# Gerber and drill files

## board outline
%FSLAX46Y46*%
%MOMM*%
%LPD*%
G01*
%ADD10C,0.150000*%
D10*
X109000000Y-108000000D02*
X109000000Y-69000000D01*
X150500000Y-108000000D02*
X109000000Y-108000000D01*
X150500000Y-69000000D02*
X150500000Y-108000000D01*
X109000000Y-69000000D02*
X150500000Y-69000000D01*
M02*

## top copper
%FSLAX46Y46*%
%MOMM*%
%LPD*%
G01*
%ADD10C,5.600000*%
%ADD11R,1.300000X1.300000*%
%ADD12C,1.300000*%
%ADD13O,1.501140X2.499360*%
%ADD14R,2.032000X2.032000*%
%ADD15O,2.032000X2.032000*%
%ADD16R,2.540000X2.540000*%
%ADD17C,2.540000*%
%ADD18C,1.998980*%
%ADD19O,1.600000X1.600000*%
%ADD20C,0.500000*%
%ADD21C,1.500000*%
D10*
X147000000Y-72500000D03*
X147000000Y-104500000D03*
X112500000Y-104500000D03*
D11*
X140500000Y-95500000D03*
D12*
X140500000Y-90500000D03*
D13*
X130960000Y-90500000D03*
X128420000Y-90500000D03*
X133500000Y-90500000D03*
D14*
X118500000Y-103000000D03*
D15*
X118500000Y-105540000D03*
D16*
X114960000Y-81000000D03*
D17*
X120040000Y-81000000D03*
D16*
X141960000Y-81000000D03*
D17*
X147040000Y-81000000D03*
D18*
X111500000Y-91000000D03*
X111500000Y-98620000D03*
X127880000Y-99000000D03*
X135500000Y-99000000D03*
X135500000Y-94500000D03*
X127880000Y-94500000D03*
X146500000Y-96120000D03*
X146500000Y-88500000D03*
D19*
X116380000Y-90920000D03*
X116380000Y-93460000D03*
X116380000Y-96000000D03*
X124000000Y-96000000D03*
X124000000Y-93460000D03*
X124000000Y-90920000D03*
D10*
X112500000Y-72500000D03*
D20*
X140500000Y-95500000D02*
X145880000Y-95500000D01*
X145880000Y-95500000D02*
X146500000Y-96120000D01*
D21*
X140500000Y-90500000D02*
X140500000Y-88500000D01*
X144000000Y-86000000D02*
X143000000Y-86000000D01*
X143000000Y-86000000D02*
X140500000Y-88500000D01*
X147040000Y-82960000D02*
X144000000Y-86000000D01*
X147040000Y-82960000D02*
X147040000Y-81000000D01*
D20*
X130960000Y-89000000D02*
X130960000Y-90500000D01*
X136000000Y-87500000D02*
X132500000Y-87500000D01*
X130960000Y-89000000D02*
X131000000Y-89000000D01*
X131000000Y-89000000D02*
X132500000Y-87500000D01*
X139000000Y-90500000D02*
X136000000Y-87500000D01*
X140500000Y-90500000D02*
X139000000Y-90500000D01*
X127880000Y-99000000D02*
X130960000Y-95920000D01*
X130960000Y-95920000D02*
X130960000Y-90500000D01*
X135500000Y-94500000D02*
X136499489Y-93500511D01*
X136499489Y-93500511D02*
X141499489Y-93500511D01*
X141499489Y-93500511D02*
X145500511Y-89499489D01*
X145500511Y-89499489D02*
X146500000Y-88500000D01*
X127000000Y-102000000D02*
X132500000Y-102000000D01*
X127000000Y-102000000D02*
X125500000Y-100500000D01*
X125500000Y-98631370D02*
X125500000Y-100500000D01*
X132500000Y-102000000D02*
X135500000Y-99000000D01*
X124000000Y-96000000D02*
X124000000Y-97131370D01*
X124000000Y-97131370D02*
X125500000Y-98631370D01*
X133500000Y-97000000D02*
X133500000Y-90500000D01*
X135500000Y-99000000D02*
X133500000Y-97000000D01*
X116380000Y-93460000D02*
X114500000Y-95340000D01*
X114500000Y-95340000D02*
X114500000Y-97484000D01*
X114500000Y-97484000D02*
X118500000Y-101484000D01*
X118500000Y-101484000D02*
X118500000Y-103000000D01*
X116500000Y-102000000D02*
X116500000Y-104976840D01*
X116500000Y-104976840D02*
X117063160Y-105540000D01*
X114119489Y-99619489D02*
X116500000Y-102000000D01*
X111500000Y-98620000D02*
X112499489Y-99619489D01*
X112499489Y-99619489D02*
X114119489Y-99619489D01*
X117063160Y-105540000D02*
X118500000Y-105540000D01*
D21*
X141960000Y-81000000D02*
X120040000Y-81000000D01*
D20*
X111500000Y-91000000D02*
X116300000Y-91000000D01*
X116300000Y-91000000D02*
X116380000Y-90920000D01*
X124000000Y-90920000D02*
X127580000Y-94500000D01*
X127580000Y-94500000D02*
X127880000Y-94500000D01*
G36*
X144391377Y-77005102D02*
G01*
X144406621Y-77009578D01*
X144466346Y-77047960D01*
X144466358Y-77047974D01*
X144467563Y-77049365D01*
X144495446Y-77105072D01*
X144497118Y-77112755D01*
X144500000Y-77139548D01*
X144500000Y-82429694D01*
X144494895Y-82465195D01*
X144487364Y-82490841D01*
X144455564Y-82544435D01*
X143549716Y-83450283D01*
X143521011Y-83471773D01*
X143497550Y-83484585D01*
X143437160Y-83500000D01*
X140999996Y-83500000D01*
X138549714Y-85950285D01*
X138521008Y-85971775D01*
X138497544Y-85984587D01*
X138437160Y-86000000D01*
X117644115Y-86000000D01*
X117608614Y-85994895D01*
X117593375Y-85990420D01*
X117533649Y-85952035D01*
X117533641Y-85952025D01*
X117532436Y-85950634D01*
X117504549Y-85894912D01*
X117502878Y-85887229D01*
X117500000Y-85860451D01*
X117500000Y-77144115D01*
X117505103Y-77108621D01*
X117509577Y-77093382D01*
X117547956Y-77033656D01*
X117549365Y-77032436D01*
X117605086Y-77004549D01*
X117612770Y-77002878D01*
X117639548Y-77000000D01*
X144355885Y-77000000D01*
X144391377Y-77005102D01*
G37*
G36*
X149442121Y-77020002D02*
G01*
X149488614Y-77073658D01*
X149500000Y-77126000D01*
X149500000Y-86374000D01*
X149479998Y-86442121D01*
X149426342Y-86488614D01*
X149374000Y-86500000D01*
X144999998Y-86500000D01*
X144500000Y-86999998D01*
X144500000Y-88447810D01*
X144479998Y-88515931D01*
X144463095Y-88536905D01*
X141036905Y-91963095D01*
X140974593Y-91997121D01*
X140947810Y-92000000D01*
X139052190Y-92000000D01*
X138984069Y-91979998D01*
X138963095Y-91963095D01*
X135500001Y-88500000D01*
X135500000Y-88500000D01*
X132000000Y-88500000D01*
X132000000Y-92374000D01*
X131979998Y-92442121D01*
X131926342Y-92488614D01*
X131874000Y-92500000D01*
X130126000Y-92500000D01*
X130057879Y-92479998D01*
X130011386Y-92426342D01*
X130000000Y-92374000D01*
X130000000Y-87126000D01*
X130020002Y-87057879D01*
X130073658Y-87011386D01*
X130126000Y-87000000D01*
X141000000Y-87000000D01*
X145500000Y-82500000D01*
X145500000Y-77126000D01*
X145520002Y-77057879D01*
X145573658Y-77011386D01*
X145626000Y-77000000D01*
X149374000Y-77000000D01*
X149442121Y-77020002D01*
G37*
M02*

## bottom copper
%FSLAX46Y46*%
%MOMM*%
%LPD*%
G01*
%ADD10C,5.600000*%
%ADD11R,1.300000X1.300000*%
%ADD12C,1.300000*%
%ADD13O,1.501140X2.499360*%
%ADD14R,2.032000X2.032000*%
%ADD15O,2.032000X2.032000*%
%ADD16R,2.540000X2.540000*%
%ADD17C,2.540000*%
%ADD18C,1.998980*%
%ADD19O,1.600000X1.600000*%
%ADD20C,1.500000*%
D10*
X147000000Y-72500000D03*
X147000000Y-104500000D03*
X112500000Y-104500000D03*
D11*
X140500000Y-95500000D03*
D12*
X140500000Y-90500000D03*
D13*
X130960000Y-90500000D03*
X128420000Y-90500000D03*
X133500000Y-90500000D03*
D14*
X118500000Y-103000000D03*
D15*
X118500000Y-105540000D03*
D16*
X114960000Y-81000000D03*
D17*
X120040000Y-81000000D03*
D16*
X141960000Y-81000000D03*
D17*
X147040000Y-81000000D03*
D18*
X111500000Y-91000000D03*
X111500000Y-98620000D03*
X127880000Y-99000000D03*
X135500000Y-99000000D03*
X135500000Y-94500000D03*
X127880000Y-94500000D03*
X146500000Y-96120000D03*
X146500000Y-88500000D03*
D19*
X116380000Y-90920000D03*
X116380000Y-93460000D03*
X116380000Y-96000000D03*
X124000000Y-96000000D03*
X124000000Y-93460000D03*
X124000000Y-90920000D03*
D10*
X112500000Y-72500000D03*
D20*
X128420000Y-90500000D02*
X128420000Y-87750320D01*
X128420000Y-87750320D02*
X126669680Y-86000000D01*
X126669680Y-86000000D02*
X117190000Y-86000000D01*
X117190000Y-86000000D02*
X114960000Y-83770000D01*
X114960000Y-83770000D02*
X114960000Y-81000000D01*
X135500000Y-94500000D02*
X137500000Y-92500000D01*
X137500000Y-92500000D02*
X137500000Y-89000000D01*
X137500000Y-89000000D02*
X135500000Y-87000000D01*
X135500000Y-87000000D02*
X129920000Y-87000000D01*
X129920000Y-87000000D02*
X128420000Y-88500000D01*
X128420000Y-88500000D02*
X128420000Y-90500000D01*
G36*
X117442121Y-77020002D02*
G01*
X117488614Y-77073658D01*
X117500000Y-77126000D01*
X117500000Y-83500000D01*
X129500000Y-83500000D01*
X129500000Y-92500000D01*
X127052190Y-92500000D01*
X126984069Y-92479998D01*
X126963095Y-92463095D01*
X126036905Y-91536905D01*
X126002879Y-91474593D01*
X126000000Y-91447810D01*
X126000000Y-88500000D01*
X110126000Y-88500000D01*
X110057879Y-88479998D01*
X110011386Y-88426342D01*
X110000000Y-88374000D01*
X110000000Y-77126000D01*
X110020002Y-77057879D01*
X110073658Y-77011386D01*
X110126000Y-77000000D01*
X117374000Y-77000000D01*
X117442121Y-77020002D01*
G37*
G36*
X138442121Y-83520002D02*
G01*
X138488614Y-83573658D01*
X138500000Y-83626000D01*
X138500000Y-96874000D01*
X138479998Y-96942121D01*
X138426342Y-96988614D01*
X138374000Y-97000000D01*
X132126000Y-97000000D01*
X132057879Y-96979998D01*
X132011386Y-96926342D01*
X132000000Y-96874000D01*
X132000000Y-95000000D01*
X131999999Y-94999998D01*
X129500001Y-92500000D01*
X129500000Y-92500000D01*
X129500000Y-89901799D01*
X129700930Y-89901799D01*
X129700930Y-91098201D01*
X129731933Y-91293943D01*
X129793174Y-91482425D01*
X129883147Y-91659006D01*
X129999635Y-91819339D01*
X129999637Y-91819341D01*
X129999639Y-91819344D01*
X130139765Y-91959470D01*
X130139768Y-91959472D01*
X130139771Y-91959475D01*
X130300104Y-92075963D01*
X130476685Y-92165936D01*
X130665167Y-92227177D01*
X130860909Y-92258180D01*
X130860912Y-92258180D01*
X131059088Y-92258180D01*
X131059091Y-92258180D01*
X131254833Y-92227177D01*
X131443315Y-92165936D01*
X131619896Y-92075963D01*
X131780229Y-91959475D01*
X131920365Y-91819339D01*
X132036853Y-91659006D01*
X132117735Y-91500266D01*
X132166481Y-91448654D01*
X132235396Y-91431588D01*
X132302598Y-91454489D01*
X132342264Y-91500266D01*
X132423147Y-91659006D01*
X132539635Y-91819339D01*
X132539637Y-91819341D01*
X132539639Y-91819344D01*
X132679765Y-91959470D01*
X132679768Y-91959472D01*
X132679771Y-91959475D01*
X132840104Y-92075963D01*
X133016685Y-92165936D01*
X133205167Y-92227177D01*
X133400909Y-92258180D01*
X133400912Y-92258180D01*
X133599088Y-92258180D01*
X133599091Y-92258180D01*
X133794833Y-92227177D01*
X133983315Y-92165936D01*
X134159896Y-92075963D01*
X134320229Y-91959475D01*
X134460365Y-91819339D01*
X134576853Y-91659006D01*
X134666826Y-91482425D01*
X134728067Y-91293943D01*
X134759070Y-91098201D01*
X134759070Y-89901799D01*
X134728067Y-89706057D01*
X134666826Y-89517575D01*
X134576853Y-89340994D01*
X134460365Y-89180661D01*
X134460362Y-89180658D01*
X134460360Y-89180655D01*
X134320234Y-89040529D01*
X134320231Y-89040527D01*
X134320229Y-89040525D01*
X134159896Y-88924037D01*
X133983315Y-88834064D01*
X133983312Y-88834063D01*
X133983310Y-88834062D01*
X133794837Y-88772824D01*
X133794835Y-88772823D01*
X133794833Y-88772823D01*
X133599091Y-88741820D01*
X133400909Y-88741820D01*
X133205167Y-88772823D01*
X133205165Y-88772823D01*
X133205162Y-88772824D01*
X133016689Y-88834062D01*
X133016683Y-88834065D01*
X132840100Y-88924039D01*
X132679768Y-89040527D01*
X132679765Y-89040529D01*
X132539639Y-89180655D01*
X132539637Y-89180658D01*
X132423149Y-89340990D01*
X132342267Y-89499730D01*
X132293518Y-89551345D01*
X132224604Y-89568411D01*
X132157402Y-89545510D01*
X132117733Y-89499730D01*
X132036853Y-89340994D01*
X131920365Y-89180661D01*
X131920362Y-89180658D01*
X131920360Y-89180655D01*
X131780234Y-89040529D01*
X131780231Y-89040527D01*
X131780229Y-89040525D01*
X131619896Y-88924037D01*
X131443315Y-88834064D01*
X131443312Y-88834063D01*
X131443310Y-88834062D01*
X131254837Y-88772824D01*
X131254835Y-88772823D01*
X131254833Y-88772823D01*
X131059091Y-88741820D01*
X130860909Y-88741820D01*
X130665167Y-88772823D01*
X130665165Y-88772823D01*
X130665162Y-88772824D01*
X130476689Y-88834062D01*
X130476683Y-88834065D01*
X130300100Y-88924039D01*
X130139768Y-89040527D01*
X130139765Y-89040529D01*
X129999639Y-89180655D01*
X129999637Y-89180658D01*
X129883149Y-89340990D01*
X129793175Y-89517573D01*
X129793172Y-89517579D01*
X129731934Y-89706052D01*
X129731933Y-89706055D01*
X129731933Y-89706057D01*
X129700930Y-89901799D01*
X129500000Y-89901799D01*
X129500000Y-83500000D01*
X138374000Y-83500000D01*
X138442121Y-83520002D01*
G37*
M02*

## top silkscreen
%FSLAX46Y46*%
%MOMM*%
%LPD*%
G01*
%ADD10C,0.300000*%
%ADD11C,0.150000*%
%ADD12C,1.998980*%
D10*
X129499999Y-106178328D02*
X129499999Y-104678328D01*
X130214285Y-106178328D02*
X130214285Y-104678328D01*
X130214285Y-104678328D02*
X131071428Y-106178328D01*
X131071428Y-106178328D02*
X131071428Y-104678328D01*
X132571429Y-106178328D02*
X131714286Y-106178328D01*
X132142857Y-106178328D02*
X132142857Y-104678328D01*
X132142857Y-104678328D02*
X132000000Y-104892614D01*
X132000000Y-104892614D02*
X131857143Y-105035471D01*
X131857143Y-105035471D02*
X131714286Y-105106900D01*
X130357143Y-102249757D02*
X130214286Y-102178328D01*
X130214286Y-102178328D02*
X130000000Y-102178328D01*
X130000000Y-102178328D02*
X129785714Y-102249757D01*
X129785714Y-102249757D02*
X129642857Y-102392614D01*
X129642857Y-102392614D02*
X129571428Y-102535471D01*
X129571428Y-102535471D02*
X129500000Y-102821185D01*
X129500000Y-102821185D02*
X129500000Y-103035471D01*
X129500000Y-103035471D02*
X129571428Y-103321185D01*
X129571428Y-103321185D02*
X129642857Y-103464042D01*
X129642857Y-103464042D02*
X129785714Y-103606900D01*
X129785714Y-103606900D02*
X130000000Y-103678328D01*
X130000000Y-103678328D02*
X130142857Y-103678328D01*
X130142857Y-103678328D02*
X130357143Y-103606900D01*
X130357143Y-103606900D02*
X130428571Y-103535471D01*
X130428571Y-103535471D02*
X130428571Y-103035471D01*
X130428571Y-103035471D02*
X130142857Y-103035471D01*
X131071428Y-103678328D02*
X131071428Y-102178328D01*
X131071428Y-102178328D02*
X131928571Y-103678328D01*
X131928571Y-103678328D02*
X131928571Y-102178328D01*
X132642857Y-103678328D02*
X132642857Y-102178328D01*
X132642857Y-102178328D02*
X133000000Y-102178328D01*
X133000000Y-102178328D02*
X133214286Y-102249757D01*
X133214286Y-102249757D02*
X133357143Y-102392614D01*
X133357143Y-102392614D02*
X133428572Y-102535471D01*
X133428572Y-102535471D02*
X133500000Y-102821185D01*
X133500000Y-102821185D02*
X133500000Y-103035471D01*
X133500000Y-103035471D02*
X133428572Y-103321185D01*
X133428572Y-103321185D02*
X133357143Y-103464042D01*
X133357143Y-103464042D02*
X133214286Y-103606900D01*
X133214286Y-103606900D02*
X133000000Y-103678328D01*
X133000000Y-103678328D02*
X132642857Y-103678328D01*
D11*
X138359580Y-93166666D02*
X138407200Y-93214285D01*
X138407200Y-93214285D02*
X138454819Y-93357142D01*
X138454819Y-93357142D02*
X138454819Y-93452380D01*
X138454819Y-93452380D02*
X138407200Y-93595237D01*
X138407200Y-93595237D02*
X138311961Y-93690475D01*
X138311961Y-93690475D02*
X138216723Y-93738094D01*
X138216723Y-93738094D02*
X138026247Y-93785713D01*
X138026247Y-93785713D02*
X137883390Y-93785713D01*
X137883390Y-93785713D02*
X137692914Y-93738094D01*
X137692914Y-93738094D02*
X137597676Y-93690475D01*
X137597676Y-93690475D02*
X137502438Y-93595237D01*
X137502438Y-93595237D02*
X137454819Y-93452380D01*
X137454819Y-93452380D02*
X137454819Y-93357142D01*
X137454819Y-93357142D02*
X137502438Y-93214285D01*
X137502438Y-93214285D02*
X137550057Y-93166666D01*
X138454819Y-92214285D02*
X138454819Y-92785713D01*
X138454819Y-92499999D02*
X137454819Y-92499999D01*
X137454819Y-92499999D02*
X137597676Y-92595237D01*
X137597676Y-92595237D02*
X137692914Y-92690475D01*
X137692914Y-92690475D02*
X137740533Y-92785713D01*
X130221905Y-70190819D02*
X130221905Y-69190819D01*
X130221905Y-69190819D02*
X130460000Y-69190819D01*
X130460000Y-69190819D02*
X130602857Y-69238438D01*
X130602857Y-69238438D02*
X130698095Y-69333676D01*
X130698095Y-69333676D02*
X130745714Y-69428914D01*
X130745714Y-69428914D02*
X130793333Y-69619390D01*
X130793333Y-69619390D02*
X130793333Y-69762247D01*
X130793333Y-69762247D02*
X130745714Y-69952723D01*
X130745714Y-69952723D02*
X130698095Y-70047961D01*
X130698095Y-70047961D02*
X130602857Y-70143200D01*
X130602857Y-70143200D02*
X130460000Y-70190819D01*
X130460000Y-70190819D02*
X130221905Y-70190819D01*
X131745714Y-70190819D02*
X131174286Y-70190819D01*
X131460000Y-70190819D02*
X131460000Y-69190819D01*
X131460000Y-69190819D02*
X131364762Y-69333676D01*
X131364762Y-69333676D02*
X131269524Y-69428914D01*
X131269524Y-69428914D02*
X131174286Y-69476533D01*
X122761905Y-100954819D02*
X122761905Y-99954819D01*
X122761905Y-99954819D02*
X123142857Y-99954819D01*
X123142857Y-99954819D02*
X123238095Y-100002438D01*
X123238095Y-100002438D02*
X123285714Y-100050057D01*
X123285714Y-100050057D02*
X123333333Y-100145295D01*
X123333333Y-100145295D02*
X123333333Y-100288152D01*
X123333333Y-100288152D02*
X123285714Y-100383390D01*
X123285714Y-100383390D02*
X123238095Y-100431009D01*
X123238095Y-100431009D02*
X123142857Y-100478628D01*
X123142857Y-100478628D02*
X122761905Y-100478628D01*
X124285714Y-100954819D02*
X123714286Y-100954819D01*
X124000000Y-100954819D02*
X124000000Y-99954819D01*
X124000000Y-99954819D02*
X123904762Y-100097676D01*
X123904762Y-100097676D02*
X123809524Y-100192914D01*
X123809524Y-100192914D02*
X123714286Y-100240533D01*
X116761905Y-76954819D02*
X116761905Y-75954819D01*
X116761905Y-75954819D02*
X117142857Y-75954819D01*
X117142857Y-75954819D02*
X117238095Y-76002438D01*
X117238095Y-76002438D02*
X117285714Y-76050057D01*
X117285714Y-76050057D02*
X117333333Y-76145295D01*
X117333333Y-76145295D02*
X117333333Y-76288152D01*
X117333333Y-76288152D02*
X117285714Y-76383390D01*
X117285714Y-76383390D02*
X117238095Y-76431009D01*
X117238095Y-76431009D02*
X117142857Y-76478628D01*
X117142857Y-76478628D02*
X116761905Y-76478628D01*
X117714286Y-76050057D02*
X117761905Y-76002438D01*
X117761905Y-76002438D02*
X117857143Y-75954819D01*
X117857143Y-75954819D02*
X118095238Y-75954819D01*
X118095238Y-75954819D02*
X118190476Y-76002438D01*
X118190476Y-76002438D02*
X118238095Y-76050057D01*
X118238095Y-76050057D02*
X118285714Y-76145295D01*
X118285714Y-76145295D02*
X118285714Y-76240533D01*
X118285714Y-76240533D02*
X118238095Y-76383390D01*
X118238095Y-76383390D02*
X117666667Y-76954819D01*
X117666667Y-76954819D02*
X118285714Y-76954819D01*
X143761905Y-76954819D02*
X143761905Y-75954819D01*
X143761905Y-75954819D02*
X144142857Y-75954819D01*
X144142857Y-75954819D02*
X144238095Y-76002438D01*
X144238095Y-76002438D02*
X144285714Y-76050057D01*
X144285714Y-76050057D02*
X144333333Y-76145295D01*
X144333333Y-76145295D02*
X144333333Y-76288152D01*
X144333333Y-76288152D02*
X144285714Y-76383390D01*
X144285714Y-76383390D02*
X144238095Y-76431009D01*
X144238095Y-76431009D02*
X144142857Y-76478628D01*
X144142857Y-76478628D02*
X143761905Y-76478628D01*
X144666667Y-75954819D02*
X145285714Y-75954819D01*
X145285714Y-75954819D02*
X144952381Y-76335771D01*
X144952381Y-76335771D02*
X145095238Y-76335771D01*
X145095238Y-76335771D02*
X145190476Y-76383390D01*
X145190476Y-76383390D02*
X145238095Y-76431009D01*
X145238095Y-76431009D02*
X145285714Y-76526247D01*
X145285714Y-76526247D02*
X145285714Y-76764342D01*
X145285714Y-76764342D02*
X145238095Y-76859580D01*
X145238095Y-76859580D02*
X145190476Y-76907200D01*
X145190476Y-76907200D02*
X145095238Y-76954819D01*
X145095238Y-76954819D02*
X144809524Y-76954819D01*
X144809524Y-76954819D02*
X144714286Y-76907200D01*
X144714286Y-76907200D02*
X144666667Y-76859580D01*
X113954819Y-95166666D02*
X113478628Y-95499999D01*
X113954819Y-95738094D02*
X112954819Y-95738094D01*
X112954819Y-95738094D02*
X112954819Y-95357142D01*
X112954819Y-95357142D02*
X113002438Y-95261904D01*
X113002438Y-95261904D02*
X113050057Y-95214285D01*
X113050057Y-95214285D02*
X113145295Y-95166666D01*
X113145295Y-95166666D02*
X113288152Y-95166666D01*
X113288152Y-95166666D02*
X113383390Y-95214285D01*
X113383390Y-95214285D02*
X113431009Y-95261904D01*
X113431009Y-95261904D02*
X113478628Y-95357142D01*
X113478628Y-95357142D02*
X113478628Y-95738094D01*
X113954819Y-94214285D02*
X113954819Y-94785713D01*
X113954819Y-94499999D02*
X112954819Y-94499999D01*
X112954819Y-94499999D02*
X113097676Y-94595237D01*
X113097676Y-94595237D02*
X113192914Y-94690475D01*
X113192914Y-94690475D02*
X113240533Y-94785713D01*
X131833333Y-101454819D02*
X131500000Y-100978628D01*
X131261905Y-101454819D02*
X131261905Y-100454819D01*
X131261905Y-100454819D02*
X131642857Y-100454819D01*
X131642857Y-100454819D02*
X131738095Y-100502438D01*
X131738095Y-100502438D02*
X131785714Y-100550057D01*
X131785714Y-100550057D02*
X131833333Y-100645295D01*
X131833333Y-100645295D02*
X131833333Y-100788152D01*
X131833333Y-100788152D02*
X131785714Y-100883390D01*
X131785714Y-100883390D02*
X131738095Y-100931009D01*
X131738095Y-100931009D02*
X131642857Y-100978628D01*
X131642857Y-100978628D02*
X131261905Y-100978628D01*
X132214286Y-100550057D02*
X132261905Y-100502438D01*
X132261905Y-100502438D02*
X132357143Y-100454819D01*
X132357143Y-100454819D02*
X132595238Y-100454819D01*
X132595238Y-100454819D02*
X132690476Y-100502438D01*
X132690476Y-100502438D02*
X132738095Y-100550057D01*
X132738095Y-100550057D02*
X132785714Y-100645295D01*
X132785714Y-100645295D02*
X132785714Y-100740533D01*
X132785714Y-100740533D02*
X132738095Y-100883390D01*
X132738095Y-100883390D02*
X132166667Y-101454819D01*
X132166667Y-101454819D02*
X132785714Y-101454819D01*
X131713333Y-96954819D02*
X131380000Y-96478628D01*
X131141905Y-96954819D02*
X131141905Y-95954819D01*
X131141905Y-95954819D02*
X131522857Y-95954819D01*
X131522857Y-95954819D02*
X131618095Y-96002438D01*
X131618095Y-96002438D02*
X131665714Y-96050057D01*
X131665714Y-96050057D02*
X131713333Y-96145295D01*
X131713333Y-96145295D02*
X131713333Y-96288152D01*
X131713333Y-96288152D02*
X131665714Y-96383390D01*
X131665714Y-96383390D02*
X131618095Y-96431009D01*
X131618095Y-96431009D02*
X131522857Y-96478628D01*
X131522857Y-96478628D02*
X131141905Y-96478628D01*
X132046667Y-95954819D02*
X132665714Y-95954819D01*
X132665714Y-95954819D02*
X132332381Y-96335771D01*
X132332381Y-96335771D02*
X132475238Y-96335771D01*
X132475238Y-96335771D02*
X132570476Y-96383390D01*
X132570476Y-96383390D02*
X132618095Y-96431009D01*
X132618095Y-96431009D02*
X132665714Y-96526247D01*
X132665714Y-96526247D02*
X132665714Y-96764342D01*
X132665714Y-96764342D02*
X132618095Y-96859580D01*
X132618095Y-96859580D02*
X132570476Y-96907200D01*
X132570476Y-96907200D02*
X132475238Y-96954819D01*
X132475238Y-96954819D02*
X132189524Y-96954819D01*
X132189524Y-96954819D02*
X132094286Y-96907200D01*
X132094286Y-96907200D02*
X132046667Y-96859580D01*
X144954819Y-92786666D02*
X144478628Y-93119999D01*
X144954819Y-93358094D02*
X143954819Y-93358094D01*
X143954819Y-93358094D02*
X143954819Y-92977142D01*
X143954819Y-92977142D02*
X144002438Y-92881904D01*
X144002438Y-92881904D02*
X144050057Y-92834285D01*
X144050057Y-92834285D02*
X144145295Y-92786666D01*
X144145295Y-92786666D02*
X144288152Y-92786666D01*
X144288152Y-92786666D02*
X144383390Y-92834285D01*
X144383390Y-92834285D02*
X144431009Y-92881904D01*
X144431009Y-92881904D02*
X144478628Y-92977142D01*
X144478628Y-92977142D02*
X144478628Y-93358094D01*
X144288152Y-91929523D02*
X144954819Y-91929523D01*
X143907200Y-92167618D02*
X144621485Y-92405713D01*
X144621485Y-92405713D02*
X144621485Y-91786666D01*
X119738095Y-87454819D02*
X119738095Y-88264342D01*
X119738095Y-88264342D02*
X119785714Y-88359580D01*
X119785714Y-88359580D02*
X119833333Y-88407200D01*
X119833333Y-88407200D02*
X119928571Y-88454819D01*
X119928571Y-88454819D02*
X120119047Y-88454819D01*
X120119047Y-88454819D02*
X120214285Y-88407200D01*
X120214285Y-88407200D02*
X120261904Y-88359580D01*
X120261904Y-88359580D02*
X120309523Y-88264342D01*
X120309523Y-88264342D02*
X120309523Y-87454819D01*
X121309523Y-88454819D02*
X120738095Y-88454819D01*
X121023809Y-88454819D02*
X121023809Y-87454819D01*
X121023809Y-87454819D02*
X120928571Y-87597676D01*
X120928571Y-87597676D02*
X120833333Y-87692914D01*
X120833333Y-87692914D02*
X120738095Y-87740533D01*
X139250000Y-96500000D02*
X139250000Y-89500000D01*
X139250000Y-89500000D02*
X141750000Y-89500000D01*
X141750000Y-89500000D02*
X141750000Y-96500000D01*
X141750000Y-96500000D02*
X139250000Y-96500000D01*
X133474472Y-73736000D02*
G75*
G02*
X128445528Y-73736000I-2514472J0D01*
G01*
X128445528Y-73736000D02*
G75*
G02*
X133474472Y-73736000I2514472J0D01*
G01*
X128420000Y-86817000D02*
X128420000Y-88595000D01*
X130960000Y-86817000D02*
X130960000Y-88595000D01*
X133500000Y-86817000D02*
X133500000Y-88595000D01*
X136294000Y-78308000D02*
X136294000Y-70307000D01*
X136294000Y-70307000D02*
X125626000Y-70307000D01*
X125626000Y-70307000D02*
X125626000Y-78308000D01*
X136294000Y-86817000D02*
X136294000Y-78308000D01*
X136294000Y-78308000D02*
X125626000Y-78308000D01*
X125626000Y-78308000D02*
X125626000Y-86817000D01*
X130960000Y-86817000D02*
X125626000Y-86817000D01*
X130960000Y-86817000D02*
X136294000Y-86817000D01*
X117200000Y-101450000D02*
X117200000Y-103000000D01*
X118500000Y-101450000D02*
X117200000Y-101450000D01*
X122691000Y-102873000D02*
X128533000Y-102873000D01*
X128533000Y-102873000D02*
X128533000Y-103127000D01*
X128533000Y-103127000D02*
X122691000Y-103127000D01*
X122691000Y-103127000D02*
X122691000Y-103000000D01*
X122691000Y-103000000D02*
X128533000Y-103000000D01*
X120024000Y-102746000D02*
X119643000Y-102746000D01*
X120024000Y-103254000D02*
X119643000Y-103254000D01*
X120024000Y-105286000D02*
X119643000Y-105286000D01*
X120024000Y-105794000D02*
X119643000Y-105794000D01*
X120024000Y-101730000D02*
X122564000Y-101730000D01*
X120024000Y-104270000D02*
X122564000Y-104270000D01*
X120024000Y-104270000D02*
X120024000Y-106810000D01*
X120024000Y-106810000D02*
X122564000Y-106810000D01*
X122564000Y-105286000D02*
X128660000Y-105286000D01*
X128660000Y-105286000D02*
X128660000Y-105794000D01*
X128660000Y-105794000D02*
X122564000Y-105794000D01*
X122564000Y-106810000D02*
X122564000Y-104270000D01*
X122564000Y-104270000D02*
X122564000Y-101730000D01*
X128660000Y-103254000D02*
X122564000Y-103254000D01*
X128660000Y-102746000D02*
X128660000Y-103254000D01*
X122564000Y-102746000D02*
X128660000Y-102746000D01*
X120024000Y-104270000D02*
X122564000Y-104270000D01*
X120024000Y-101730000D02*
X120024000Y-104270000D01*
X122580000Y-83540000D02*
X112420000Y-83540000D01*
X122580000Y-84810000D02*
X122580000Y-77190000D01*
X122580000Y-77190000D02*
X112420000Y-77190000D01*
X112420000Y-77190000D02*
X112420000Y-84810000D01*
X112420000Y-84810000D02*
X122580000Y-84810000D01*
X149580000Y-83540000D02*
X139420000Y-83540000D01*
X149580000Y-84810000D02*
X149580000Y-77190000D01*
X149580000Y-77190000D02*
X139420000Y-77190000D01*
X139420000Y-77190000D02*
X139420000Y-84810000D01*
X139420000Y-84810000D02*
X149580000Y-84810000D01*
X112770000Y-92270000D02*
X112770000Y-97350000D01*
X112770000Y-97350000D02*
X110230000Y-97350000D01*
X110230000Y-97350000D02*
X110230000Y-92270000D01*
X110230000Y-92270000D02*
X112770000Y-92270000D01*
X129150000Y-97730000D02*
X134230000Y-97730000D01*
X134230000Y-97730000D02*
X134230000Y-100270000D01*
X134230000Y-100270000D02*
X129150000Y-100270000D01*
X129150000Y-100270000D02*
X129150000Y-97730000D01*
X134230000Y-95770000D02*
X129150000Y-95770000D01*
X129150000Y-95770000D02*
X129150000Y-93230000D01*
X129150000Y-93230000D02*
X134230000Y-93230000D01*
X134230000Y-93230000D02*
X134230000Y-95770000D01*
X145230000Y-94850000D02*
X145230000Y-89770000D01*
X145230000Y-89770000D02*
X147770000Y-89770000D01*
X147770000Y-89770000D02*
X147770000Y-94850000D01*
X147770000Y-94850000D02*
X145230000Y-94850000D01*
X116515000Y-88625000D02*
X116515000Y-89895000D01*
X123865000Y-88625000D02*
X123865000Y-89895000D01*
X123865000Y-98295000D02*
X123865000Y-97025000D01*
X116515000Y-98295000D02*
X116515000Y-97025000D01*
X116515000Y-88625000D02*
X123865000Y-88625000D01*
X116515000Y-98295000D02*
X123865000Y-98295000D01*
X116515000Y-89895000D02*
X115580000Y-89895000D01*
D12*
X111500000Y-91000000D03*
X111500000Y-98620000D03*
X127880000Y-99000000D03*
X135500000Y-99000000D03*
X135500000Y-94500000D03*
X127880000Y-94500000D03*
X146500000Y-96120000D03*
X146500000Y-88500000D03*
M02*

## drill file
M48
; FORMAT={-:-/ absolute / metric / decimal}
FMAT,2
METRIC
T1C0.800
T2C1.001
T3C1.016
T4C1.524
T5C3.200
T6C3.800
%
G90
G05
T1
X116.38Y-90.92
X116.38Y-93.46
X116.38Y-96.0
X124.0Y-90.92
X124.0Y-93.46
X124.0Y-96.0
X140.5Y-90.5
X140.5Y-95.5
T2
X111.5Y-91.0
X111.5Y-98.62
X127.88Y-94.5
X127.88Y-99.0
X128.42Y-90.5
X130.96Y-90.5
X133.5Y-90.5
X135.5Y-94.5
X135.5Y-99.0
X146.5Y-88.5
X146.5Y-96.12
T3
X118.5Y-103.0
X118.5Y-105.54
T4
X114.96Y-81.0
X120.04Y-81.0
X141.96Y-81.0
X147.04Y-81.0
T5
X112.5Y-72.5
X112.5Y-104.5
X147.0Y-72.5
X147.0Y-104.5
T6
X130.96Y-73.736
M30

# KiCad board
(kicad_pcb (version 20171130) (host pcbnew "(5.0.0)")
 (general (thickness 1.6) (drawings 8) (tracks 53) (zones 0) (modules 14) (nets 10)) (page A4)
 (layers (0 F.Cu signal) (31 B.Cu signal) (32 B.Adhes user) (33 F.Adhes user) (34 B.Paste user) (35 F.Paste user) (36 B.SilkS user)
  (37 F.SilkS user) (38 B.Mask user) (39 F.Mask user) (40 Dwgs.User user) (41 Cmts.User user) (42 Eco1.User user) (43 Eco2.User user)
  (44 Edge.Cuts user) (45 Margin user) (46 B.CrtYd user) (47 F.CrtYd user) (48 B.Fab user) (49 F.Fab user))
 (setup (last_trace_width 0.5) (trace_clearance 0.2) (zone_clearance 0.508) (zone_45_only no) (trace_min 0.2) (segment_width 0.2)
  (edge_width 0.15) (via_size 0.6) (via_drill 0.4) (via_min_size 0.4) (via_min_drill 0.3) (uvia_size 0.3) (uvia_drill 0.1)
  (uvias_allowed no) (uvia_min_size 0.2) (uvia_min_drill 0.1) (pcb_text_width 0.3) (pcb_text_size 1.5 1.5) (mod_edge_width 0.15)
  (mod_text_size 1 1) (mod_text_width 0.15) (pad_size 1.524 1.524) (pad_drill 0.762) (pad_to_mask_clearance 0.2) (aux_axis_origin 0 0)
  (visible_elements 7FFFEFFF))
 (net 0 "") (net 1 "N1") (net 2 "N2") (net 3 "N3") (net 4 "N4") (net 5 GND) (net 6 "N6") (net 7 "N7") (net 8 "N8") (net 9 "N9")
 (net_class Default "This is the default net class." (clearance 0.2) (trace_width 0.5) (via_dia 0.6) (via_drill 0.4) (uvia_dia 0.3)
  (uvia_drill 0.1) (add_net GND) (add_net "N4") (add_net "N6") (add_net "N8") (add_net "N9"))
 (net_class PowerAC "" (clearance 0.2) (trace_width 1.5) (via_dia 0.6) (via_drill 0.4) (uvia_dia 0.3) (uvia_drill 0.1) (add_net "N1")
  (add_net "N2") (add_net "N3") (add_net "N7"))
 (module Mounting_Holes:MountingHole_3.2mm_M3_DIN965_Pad (layer F.Cu) (at 147 72.5)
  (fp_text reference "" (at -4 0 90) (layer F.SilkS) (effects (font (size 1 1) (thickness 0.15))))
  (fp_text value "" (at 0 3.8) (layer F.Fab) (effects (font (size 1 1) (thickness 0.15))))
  (pad 1 thru_hole circle (at 0 0) (size 5.6 5.6) (drill 3.2) (layers *.Cu *.Mask)))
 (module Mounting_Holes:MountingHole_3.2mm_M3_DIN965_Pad (layer F.Cu) (at 147 104.5)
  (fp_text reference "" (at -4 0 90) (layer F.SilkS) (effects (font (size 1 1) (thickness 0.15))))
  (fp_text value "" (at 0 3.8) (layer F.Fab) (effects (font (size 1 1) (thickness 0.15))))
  (pad 1 thru_hole circle (at 0 0) (size 5.6 5.6) (drill 3.2) (layers *.Cu *.Mask)))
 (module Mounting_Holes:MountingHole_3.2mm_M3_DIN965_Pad (layer F.Cu) (at 112.5 104.5)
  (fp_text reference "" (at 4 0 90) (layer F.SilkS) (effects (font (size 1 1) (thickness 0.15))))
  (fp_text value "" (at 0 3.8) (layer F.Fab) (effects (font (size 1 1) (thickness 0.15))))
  (pad 1 thru_hole circle (at 0 0) (size 5.6 5.6) (drill 3.2) (layers *.Cu *.Mask)))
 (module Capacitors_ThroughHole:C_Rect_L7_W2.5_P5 (layer F.Cu) (at 140.5 95.5 90)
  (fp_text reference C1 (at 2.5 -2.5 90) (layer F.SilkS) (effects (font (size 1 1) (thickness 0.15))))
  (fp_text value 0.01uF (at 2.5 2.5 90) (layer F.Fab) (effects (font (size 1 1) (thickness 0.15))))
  (fp_line (start -1 -1.25) (end 6 -1.25) (layer F.SilkS) (width 0.15))
  (fp_line (start 6 -1.25) (end 6 1.25) (layer F.SilkS) (width 0.15))
  (fp_line (start 6 1.25) (end -1 1.25) (layer F.SilkS) (width 0.15))
  (fp_line (start -1 1.25) (end -1 -1.25) (layer F.SilkS) (width 0.15))
  (pad 1 thru_hole rect (at 0 0 90) (size 1.3 1.3) (drill 0.8) (layers *.Cu *.Mask) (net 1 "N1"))
  (pad 2 thru_hole circle (at 5 0 90) (size 1.3 1.3) (drill 0.8) (layers *.Cu *.Mask) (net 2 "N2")))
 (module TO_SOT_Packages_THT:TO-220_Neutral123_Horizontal (layer F.Cu) (at 130.96 90.5)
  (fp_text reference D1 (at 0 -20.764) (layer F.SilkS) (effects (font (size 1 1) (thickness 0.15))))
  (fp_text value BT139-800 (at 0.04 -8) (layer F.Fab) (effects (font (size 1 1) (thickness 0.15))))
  (fp_circle (center 0 -16.764) (end 1.778 -14.986) (layer F.SilkS) (width 0.15))
  (fp_line (start -2.54 -3.683) (end -2.54 -1.905) (layer F.SilkS) (width 0.15))
  (fp_line (start 0 -3.683) (end 0 -1.905) (layer F.SilkS) (width 0.15))
  (fp_line (start 2.54 -3.683) (end 2.54 -1.905) (layer F.SilkS) (width 0.15))
  (fp_line (start 5.334 -12.192) (end 5.334 -20.193) (layer F.SilkS) (width 0.15))
  (fp_line (start 5.334 -20.193) (end -5.334 -20.193) (layer F.SilkS) (width 0.15))
  (fp_line (start -5.334 -20.193) (end -5.334 -12.192) (layer F.SilkS) (width 0.15))
  (fp_line (start 5.334 -3.683) (end 5.334 -12.192) (layer F.SilkS) (width 0.15))
  (fp_line (start 5.334 -12.192) (end -5.334 -12.192) (layer F.SilkS) (width 0.15))
  (fp_line (start -5.334 -12.192) (end -5.334 -3.683) (layer F.SilkS) (width 0.15))
  (fp_line (start 0 -3.683) (end -5.334 -3.683) (layer F.SilkS) (width 0.15))
  (fp_line (start 0 -3.683) (end 5.334 -3.683) (layer F.SilkS) (width 0.15))
  (pad 2 thru_hole oval (at 0 0 90) (size 2.49936 1.50114) (drill 1.00076) (layers *.Cu *.Mask) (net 2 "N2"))
  (pad 1 thru_hole oval (at -2.54 0 90) (size 2.49936 1.50114) (drill 1.00076) (layers *.Cu *.Mask) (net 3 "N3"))
  (pad 3 thru_hole oval (at 2.54 0 90) (size 2.49936 1.50114) (drill 1.00076) (layers *.Cu *.Mask) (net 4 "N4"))
  (pad "" np_thru_hole circle (at 0 -16.764 90) (size 3.79984 3.79984) (drill 3.79984) (layers *.Cu *.Mask)))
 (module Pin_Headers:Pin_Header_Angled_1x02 (layer F.Cu) (at 118.5 103)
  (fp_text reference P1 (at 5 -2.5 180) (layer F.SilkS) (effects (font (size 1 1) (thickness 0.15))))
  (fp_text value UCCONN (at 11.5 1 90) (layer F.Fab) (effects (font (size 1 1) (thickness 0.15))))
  (fp_line (start -1.3 -1.55) (end -1.3 0) (layer F.SilkS) (width 0.15))
  (fp_line (start 0 -1.55) (end -1.3 -1.55) (layer F.SilkS) (width 0.15))
  (fp_line (start 4.191 -0.127) (end 10.033 -0.127) (layer F.SilkS) (width 0.15))
  (fp_line (start 10.033 -0.127) (end 10.033 0.127) (layer F.SilkS) (width 0.15))
  (fp_line (start 10.033 0.127) (end 4.191 0.127) (layer F.SilkS) (width 0.15))
  (fp_line (start 4.191 0.127) (end 4.191 0) (layer F.SilkS) (width 0.15))
  (fp_line (start 4.191 0) (end 10.033 0) (layer F.SilkS) (width 0.15))
  (fp_line (start 1.524 -0.254) (end 1.143 -0.254) (layer F.SilkS) (width 0.15))
  (fp_line (start 1.524 0.254) (end 1.143 0.254) (layer F.SilkS) (width 0.15))
  (fp_line (start 1.524 2.286) (end 1.143 2.286) (layer F.SilkS) (width 0.15))
  (fp_line (start 1.524 2.794) (end 1.143 2.794) (layer F.SilkS) (width 0.15))
  (fp_line (start 1.524 -1.27) (end 4.064 -1.27) (layer F.SilkS) (width 0.15))
  (fp_line (start 1.524 1.27) (end 4.064 1.27) (layer F.SilkS) (width 0.15))
  (fp_line (start 1.524 1.27) (end 1.524 3.81) (layer F.SilkS) (width 0.15))
  (fp_line (start 1.524 3.81) (end 4.064 3.81) (layer F.SilkS) (width 0.15))
  (fp_line (start 4.064 2.286) (end 10.16 2.286) (layer F.SilkS) (width 0.15))
  (fp_line (start 10.16 2.286) (end 10.16 2.794) (layer F.SilkS) (width 0.15))
  (fp_line (start 10.16 2.794) (end 4.064 2.794) (layer F.SilkS) (width 0.15))
  (fp_line (start 4.064 3.81) (end 4.064 1.27) (layer F.SilkS) (width 0.15))
  (fp_line (start 4.064 1.27) (end 4.064 -1.27) (layer F.SilkS) (width 0.15))
  (fp_line (start 10.16 0.254) (end 4.064 0.254) (layer F.SilkS) (width 0.15))
  (fp_line (start 10.16 -0.254) (end 10.16 0.254) (layer F.SilkS) (width 0.15))
  (fp_line (start 4.064 -0.254) (end 10.16 -0.254) (layer F.SilkS) (width 0.15))
  (fp_line (start 1.524 1.27) (end 4.064 1.27) (layer F.SilkS) (width 0.15))
  (fp_line (start 1.524 -1.27) (end 1.524 1.27) (layer F.SilkS) (width 0.15))
  (pad 1 thru_hole rect (at 0 0) (size 2.032 2.032) (drill 1.016) (layers *.Cu *.Mask) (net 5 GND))
  (pad 2 thru_hole oval (at 0 2.54) (size 2.032 2.032) (drill 1.016) (layers *.Cu *.Mask) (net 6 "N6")))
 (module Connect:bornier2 (layer F.Cu) (at 117.5 81)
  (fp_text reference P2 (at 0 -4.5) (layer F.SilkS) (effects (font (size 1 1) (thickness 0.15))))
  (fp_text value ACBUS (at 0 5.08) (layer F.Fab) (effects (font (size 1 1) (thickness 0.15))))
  (fp_line (start 5.08 2.54) (end -5.08 2.54) (layer F.SilkS) (width 0.15))
  (fp_line (start 5.08 3.81) (end 5.08 -3.81) (layer F.SilkS) (width 0.15))
  (fp_line (start 5.08 -3.81) (end -5.08 -3.81) (layer F.SilkS) (width 0.15))
  (fp_line (start -5.08 -3.81) (end -5.08 3.81) (layer F.SilkS) (width 0.15))
  (fp_line (start -5.08 3.81) (end 5.08 3.81) (layer F.SilkS) (width 0.15))
  (pad 1 thru_hole rect (at -2.54 0) (size 2.54 2.54) (drill 1.524) (layers *.Cu *.Mask) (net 3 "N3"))
  (pad 2 thru_hole circle (at 2.54 0) (size 2.54 2.54) (drill 1.524) (layers *.Cu *.Mask) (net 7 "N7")))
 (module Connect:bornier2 (layer F.Cu) (at 144.5 81)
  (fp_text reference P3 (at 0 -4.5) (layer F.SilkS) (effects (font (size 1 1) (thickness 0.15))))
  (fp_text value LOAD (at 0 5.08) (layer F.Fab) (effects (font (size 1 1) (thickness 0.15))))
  (fp_line (start 5.08 2.54) (end -5.08 2.54) (layer F.SilkS) (width 0.15))
  (fp_line (start 5.08 3.81) (end 5.08 -3.81) (layer F.SilkS) (width 0.15))
  (fp_line (start 5.08 -3.81) (end -5.08 -3.81) (layer F.SilkS) (width 0.15))
  (fp_line (start -5.08 -3.81) (end -5.08 3.81) (layer F.SilkS) (width 0.15))
  (fp_line (start -5.08 3.81) (end 5.08 3.81) (layer F.SilkS) (width 0.15))
  (pad 1 thru_hole rect (at -2.54 0) (size 2.54 2.54) (drill 1.524) (layers *.Cu *.Mask) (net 7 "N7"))
  (pad 2 thru_hole circle (at 2.54 0) (size 2.54 2.54) (drill 1.524) (layers *.Cu *.Mask) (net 2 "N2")))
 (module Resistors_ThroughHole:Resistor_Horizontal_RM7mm (layer F.Cu) (at 111.5 91 270)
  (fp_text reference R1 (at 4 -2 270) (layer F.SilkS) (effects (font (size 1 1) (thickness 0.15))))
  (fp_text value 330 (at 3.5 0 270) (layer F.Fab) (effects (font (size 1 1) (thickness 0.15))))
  (fp_line (start 1.27 -1.27) (end 6.35 -1.27) (layer F.SilkS) (width 0.15))
  (fp_line (start 6.35 -1.27) (end 6.35 1.27) (layer F.SilkS) (width 0.15))
  (fp_line (start 6.35 1.27) (end 1.27 1.27) (layer F.SilkS) (width 0.15))
  (fp_line (start 1.27 1.27) (end 1.27 -1.27) (layer F.SilkS) (width 0.15))
  (pad 1 thru_hole circle (at 0 0 270) (size 1.99898 1.99898) (drill 1.00076) (layers *.Cu *.SilkS *.Mask) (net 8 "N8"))
  (pad 2 thru_hole circle (at 7.62 0 270) (size 1.99898 1.99898) (drill 1.00076) (layers *.Cu *.SilkS *.Mask) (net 6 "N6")))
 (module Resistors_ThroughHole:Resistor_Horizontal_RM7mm (layer F.Cu) (at 127.88 99)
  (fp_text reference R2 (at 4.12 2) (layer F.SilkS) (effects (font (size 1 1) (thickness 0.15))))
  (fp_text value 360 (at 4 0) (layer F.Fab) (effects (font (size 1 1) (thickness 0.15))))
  (fp_line (start 1.27 -1.27) (end 6.35 -1.27) (layer F.SilkS) (width 0.15))
  (fp_line (start 6.35 -1.27) (end 6.35 1.27) (layer F.SilkS) (width 0.15))
  (fp_line (start 6.35 1.27) (end 1.27 1.27) (layer F.SilkS) (width 0.15))
  (fp_line (start 1.27 1.27) (end 1.27 -1.27) (layer F.SilkS) (width 0.15))
  (pad 1 thru_hole circle (at 0 0) (size 1.99898 1.99898) (drill 1.00076) (layers *.Cu *.SilkS *.Mask) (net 2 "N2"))
  (pad 2 thru_hole circle (at 7.62 0) (size 1.99898 1.99898) (drill 1.00076) (layers *.Cu *.SilkS *.Mask) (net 4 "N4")))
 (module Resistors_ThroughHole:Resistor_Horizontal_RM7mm (layer F.Cu) (at 135.5 94.5 180)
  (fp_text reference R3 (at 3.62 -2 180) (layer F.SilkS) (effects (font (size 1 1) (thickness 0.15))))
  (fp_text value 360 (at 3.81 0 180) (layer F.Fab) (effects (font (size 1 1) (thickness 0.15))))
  (fp_line (start 1.27 -1.27) (end 6.35 -1.27) (layer F.SilkS) (width 0.15))
  (fp_line (start 6.35 -1.27) (end 6.35 1.27) (layer F.SilkS) (width 0.15))
  (fp_line (start 6.35 1.27) (end 1.27 1.27) (layer F.SilkS) (width 0.15))
  (fp_line (start 1.27 1.27) (end 1.27 -1.27) (layer F.SilkS) (width 0.15))
  (pad 1 thru_hole circle (at 0 0 180) (size 1.99898 1.99898) (drill 1.00076) (layers *.Cu *.SilkS *.Mask) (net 3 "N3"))
  (pad 2 thru_hole circle (at 7.62 0 180) (size 1.99898 1.99898) (drill 1.00076) (layers *.Cu *.SilkS *.Mask) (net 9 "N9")))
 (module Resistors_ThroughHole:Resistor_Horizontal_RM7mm (layer F.Cu) (at 146.5 96.12 90)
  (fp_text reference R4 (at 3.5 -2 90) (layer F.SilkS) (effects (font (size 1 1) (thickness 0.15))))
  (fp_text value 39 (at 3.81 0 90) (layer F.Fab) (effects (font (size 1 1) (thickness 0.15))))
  (fp_line (start 1.27 -1.27) (end 6.35 -1.27) (layer F.SilkS) (width 0.15))
  (fp_line (start 6.35 -1.27) (end 6.35 1.27) (layer F.SilkS) (width 0.15))
  (fp_line (start 6.35 1.27) (end 1.27 1.27) (layer F.SilkS) (width 0.15))
  (fp_line (start 1.27 1.27) (end 1.27 -1.27) (layer F.SilkS) (width 0.15))
  (pad 1 thru_hole circle (at 0 0 90) (size 1.99898 1.99898) (drill 1.00076) (layers *.Cu *.SilkS *.Mask) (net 1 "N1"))
  (pad 2 thru_hole circle (at 7.62 0 90) (size 1.99898 1.99898) (drill 1.00076) (layers *.Cu *.SilkS *.Mask) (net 3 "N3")))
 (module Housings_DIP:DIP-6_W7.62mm (layer F.Cu) (at 116.38 90.92)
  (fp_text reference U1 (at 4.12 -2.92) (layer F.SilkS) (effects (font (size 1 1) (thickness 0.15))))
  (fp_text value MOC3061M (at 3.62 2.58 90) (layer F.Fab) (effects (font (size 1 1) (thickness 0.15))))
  (fp_line (start 0.135 -2.295) (end 0.135 -1.025) (layer F.SilkS) (width 0.15))
  (fp_line (start 7.485 -2.295) (end 7.485 -1.025) (layer F.SilkS) (width 0.15))
  (fp_line (start 7.485 7.375) (end 7.485 6.105) (layer F.SilkS) (width 0.15))
  (fp_line (start 0.135 7.375) (end 0.135 6.105) (layer F.SilkS) (width 0.15))
  (fp_line (start 0.135 -2.295) (end 7.485 -2.295) (layer F.SilkS) (width 0.15))
  (fp_line (start 0.135 7.375) (end 7.485 7.375) (layer F.SilkS) (width 0.15))
  (fp_line (start 0.135 -1.025) (end -0.8 -1.025) (layer F.SilkS) (width 0.15))
  (pad 1 thru_hole oval (at 0 0) (size 1.6 1.6) (drill 0.8) (layers *.Cu *.Mask) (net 8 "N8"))
  (pad 2 thru_hole oval (at 0 2.54) (size 1.6 1.6) (drill 0.8) (layers *.Cu *.Mask) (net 5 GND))
  (pad 3 thru_hole oval (at 0 5.08) (size 1.6 1.6) (drill 0.8) (layers *.Cu *.Mask))
  (pad 4 thru_hole oval (at 7.62 5.08) (size 1.6 1.6) (drill 0.8) (layers *.Cu *.Mask) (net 4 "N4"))
  (pad 5 thru_hole oval (at 7.62 2.54) (size 1.6 1.6) (drill 0.8) (layers *.Cu *.Mask))
  (pad 6 thru_hole oval (at 7.62 0) (size 1.6 1.6) (drill 0.8) (layers *.Cu *.Mask) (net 9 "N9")))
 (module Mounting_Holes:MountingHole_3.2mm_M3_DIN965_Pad (layer F.Cu) (at 112.5 72.5)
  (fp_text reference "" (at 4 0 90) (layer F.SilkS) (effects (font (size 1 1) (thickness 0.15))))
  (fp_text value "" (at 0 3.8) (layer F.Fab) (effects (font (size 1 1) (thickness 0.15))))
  (pad 1 thru_hole circle (at 0 0) (size 5.6 5.6) (drill 3.2) (layers *.Cu *.Mask)))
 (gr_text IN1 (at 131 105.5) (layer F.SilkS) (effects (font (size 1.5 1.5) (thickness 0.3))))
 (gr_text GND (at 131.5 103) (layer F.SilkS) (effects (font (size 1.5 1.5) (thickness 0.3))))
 (gr_line (start 109 108) (end 109 69) (layer Edge.Cuts) (width 0.15))
 (gr_line (start 150.5 108) (end 109 108) (layer Edge.Cuts) (width 0.15))
 (gr_line (start 150.5 69) (end 150.5 108) (layer Edge.Cuts) (width 0.15))
 (gr_line (start 109 69) (end 150.5 69) (layer Edge.Cuts) (width 0.15))
 (segment (start 140.5 95.5) (end 145.88 95.5) (width 0.5) (layer F.Cu) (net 1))
 (segment (start 145.88 95.5) (end 146.5 96.12) (width 0.5) (layer F.Cu) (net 1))
 (segment (start 140.5 90.5) (end 140.5 88.5) (width 1.5) (layer F.Cu) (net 2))
 (segment (start 144 86) (end 143 86) (width 1.5) (layer F.Cu) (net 2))
 (segment (start 143 86) (end 140.5 88.5) (width 1.5) (layer F.Cu) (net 2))
 (segment (start 147.04 82.96) (end 144 86) (width 1.5) (layer F.Cu) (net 2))
 (segment (start 147.04 82.96) (end 147.04 81) (width 1.5) (layer F.Cu) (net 2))
 (segment (start 130.96 89) (end 130.96 90.5) (width 0.5) (layer F.Cu) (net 2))
 (segment (start 136 87.5) (end 132.5 87.5) (width 0.5) (layer F.Cu) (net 2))
 (segment (start 130.96 89) (end 131 89) (width 0.5) (layer F.Cu) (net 2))
 (segment (start 131 89) (end 132.5 87.5) (width 0.5) (layer F.Cu) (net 2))
 (segment (start 139 90.5) (end 136 87.5) (width 0.5) (layer F.Cu) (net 2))
 (segment (start 140.5 90.5) (end 139 90.5) (width 0.5) (layer F.Cu) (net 2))
 (segment (start 127.88 99) (end 130.96 95.92) (width 0.5) (layer F.Cu) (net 2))
 (segment (start 130.96 95.92) (end 130.96 90.5) (width 0.5) (layer F.Cu) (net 2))
 (segment (start 128.42 90.5) (end 128.42 87.75032) (width 1.5) (layer B.Cu) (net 3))
 (segment (start 128.42 87.75032) (end 126.66968 86) (width 1.5) (layer B.Cu) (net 3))
 (segment (start 126.66968 86) (end 117.19 86) (width 1.5) (layer B.Cu) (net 3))
 (segment (start 117.19 86) (end 114.96 83.77) (width 1.5) (layer B.Cu) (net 3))
 (segment (start 114.96 83.77) (end 114.96 81) (width 1.5) (layer B.Cu) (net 3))
 (segment (start 135.5 94.5) (end 137.5 92.5) (width 1.5) (layer B.Cu) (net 3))
 (segment (start 137.5 92.5) (end 137.5 89) (width 1.5) (layer B.Cu) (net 3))
 (segment (start 137.5 89) (end 135.5 87) (width 1.5) (layer B.Cu) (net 3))
 (segment (start 135.5 87) (end 129.92 87) (width 1.5) (layer B.Cu) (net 3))
 (segment (start 129.92 87) (end 128.42 88.5) (width 1.5) (layer B.Cu) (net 3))
 (segment (start 128.42 88.5) (end 128.42 90.5) (width 1.5) (layer B.Cu) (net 3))
 (segment (start 135.5 94.5) (end 136.499489 93.500511) (width 0.5) (layer F.Cu) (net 3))
 (segment (start 136.499489 93.500511) (end 141.499489 93.500511) (width 0.5) (layer F.Cu) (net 3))
 (segment (start 141.499489 93.500511) (end 145.500511 89.499489) (width 0.5) (layer F.Cu) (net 3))
 (segment (start 145.500511 89.499489) (end 146.5 88.5) (width 0.5) (layer F.Cu) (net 3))
 (segment (start 127 102) (end 132.5 102) (width 0.5) (layer F.Cu) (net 4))
 (segment (start 127 102) (end 125.5 100.5) (width 0.5) (layer F.Cu) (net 4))
 (segment (start 125.5 98.63137) (end 125.5 100.5) (width 0.5) (layer F.Cu) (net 4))
 (segment (start 132.5 102) (end 135.5 99) (width 0.5) (layer F.Cu) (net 4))
 (segment (start 124 96) (end 124 97.13137) (width 0.5) (layer F.Cu) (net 4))
 (segment (start 124 97.13137) (end 125.5 98.63137) (width 0.5) (layer F.Cu) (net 4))
 (segment (start 133.5 97) (end 133.5 90.5) (width 0.5) (layer F.Cu) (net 4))
 (segment (start 135.5 99) (end 133.5 97) (width 0.5) (layer F.Cu) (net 4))
 (segment (start 116.38 93.46) (end 114.5 95.34) (width 0.5) (layer F.Cu) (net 5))
 (segment (start 114.5 95.34) (end 114.5 97.484) (width 0.5) (layer F.Cu) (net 5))
 (segment (start 114.5 97.484) (end 118.5 101.484) (width 0.5) (layer F.Cu) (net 5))
 (segment (start 118.5 101.484) (end 118.5 103) (width 0.5) (layer F.Cu) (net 5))
 (segment (start 116.5 102) (end 116.5 104.97684) (width 0.5) (layer F.Cu) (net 6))
 (segment (start 116.5 104.97684) (end 117.06316 105.54) (width 0.5) (layer F.Cu) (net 6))
 (segment (start 114.119489 99.619489) (end 116.5 102) (width 0.5) (layer F.Cu) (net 6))
 (segment (start 111.5 98.62) (end 112.499489 99.619489) (width 0.5) (layer F.Cu) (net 6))
 (segment (start 112.499489 99.619489) (end 114.119489 99.619489) (width 0.5) (layer F.Cu) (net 6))
 (segment (start 117.06316 105.54) (end 118.5 105.54) (width 0.5) (layer F.Cu) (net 6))
 (segment (start 141.96 81) (end 120.04 81) (width 1.5) (layer F.Cu) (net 7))
 (segment (start 111.5 91) (end 116.3 91) (width 0.5) (layer F.Cu) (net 8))
 (segment (start 116.3 91) (end 116.38 90.92) (width 0.5) (layer F.Cu) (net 8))
 (segment (start 124 90.92) (end 127.58 94.5) (width 0.5) (layer F.Cu) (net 9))
 (segment (start 127.58 94.5) (end 127.88 94.5) (width 0.5) (layer F.Cu) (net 9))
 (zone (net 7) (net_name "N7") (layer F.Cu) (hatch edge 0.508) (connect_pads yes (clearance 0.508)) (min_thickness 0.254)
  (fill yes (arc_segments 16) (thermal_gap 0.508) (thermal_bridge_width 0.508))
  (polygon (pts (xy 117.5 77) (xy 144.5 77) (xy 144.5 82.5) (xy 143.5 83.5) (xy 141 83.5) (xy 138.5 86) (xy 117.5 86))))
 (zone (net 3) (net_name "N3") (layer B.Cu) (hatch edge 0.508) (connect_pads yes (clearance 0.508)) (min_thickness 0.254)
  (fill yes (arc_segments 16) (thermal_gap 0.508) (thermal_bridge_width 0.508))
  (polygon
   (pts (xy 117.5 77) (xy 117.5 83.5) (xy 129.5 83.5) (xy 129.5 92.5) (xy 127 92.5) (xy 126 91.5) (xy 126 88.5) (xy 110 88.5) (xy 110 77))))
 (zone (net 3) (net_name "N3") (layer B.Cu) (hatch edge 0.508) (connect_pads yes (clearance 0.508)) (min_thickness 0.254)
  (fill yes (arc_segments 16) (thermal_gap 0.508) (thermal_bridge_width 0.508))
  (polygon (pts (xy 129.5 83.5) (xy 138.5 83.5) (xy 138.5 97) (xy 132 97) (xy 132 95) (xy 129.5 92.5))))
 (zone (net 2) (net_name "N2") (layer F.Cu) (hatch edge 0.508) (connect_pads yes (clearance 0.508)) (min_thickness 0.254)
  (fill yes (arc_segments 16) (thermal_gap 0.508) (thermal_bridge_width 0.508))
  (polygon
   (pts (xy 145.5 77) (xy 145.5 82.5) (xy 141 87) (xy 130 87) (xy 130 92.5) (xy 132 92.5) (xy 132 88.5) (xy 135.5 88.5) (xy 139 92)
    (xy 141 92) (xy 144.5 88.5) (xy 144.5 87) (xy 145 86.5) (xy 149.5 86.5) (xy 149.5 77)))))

